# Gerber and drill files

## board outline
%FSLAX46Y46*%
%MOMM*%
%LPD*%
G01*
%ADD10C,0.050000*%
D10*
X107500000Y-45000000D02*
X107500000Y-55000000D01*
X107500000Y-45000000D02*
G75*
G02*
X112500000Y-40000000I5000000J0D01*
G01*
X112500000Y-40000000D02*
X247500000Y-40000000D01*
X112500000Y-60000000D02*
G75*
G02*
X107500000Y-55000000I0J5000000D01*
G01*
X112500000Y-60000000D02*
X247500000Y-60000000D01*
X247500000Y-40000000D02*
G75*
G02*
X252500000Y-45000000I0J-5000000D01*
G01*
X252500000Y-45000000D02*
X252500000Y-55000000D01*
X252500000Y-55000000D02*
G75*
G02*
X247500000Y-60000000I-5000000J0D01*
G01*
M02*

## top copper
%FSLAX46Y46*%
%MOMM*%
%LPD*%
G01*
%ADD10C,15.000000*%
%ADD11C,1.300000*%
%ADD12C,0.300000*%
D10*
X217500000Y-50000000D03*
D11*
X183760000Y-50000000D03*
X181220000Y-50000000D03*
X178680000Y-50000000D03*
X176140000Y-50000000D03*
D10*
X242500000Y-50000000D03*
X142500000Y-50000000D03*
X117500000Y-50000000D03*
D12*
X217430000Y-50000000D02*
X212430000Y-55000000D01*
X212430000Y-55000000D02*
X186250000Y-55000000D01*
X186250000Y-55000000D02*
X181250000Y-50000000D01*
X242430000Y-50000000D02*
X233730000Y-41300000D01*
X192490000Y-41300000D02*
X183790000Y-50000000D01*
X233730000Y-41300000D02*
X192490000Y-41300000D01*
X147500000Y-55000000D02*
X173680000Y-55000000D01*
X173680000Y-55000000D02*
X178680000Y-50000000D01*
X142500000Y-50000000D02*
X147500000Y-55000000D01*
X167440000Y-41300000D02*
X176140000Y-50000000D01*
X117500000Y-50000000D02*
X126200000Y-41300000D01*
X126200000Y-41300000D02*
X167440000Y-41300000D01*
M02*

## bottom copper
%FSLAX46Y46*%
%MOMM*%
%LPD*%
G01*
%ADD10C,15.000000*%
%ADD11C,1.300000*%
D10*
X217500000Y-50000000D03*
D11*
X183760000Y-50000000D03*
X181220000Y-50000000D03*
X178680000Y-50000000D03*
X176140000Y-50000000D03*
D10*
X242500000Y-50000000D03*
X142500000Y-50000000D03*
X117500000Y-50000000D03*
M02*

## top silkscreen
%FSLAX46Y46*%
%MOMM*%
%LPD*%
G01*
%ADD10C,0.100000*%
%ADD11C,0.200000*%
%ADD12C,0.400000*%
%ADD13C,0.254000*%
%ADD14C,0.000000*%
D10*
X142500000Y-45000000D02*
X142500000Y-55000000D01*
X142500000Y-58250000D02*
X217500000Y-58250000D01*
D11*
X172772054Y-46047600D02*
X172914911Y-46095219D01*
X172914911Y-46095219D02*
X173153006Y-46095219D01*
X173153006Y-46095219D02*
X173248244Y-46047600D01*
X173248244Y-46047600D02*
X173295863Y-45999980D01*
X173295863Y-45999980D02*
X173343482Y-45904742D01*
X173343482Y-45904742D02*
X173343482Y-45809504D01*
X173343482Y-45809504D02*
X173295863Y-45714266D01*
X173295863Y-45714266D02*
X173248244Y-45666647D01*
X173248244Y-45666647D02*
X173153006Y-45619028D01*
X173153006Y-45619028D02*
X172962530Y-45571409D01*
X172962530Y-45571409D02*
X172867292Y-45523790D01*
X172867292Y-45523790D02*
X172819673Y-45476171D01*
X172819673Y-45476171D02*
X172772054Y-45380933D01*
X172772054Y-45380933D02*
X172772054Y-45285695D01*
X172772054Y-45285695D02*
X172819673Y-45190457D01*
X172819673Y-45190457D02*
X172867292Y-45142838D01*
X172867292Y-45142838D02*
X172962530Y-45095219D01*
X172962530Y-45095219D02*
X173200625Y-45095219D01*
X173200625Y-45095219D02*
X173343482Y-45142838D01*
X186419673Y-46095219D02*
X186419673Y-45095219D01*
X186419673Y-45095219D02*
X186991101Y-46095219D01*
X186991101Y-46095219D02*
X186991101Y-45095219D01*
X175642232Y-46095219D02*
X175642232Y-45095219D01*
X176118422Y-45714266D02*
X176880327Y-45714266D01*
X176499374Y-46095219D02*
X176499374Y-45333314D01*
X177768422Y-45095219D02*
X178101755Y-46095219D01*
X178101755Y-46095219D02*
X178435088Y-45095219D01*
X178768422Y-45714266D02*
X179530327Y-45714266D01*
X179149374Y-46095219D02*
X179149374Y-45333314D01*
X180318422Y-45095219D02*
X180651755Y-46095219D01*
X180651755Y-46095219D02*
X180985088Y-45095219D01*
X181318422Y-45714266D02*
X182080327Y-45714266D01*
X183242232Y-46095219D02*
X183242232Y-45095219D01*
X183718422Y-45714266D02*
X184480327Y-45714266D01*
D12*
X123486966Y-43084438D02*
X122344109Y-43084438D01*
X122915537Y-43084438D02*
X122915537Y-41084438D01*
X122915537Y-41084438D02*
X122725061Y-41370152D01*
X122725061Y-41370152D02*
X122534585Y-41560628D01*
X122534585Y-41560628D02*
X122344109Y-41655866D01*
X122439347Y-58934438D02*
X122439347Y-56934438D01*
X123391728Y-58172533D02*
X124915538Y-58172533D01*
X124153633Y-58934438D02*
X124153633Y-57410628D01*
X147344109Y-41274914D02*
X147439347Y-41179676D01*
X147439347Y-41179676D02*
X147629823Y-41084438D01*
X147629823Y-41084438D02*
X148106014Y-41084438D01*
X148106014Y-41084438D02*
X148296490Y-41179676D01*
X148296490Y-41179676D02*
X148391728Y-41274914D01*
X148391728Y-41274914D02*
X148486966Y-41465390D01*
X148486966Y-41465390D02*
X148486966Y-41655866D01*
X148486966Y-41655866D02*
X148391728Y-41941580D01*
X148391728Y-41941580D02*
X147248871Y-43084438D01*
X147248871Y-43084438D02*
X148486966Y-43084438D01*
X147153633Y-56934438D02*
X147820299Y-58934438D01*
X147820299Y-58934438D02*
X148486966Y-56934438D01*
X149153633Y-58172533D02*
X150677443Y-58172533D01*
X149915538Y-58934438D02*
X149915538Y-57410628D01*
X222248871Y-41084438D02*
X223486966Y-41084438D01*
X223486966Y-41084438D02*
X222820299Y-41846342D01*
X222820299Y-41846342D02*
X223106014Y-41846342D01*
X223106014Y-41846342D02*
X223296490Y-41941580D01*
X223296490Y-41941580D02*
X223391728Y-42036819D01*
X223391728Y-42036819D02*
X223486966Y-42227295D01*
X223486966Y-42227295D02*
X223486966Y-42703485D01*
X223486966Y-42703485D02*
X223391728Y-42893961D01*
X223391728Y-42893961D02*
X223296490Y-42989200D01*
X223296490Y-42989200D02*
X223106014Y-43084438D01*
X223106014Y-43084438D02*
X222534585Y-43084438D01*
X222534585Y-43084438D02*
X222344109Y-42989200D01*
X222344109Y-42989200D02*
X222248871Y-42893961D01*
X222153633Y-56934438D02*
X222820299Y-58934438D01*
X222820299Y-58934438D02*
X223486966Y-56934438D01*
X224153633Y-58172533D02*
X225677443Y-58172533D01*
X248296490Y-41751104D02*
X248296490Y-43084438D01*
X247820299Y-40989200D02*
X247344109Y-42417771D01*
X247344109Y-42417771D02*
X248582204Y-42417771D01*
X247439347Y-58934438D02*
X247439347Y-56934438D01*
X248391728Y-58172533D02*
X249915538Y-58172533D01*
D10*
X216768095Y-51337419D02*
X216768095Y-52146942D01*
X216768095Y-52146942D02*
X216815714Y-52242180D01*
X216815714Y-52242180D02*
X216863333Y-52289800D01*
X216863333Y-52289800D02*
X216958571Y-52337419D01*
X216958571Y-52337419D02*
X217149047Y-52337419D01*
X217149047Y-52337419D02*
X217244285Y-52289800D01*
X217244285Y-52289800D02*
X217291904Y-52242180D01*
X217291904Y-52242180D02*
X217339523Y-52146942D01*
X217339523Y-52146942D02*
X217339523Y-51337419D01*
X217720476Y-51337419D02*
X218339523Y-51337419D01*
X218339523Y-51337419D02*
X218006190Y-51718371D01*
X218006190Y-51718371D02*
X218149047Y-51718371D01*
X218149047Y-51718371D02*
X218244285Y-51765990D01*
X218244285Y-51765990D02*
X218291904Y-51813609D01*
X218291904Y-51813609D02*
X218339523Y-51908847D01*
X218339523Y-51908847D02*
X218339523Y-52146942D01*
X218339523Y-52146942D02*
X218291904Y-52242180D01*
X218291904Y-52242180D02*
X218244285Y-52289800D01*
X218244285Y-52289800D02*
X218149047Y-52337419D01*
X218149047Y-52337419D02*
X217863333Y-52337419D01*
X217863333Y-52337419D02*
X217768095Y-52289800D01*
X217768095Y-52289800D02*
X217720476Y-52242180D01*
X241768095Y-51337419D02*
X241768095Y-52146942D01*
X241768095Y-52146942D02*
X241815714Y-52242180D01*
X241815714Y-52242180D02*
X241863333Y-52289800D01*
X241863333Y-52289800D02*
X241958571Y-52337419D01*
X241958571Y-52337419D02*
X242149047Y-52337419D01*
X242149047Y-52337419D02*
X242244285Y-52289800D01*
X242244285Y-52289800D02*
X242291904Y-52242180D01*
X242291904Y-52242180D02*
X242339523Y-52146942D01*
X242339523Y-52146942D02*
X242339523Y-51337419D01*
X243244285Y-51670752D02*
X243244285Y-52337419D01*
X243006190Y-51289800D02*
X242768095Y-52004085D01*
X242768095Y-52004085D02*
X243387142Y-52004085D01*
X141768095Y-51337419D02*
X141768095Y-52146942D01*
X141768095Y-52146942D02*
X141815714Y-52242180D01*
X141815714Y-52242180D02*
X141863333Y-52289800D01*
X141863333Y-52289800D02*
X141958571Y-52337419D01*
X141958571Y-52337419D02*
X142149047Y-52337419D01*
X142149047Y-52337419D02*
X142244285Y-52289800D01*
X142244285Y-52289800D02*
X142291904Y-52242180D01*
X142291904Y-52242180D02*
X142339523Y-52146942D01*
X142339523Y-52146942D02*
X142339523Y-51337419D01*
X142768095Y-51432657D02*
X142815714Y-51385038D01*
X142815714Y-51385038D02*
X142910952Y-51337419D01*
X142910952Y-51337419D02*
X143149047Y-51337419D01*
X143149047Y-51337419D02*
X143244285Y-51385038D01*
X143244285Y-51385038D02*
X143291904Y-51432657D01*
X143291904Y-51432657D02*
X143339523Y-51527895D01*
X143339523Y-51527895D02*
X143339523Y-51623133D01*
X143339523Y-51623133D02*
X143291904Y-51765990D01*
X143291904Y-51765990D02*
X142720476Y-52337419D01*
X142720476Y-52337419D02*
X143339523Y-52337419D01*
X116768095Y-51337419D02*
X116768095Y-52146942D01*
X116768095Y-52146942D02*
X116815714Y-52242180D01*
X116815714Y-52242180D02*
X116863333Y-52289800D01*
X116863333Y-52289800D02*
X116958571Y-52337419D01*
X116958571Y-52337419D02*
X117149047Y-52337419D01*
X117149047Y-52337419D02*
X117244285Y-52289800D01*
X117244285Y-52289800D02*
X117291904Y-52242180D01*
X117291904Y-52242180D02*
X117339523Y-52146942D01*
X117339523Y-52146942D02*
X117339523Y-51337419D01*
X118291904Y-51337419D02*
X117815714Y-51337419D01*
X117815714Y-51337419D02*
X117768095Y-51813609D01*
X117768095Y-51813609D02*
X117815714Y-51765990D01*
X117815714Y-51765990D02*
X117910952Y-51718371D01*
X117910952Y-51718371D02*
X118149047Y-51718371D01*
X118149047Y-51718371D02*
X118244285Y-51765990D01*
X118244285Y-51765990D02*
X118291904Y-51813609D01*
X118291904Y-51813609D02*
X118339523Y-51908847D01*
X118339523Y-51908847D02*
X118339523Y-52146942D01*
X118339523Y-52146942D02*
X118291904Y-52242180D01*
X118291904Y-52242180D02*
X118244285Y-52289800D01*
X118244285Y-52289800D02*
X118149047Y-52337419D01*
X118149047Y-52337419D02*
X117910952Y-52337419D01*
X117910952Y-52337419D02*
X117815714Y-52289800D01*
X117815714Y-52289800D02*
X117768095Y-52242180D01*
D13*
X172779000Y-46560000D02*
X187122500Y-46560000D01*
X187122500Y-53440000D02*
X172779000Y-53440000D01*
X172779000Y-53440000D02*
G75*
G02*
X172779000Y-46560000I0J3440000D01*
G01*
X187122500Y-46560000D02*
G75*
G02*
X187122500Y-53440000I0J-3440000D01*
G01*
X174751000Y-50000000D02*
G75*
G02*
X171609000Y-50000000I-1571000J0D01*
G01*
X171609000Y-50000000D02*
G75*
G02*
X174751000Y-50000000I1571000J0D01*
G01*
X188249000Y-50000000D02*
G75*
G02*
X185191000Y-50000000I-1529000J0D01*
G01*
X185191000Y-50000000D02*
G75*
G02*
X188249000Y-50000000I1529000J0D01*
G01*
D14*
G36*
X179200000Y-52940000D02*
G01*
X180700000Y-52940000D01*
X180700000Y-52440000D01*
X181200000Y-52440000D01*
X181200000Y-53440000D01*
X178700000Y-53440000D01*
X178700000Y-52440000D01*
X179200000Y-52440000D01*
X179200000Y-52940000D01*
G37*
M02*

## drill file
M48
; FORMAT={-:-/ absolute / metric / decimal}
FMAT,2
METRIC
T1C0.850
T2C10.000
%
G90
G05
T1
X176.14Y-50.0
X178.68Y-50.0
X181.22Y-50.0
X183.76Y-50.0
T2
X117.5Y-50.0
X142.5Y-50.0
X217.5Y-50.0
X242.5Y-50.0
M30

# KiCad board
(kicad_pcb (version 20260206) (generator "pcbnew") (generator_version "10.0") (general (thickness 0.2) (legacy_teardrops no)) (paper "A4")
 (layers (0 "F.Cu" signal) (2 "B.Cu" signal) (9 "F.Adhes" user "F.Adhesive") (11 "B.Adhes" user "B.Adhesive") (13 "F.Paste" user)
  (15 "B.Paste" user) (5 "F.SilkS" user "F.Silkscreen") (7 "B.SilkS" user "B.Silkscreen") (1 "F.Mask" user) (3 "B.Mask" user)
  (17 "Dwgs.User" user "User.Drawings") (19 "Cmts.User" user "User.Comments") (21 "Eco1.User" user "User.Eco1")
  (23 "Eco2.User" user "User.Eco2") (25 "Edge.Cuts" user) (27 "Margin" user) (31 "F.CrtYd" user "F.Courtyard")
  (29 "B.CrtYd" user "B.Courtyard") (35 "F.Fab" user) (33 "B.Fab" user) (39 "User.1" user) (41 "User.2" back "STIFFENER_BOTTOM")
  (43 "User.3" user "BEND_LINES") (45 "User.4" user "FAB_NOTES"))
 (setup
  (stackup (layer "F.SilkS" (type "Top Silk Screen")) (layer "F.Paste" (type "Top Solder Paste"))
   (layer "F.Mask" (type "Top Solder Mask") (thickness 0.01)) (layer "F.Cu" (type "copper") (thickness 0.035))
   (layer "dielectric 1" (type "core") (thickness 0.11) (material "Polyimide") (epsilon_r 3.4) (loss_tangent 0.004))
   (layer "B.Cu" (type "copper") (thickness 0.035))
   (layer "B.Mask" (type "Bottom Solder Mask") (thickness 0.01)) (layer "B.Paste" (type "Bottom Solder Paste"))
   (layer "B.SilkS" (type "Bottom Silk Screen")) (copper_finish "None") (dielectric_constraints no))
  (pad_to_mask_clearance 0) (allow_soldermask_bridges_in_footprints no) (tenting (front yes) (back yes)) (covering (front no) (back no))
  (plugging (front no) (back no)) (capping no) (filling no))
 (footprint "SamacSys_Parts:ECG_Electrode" (layer "F.Cu") (at 217.53 52.38)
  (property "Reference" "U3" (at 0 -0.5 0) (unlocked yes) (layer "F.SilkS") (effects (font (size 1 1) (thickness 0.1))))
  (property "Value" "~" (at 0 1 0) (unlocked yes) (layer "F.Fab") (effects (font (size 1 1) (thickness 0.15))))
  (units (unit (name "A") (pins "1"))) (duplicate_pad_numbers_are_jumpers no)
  (pad "1" thru_hole circle (at -0.03 -2.38) (size 15 15) (drill 10) (layers "*.Cu" "*.Mask") (remove_unused_layers no) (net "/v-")))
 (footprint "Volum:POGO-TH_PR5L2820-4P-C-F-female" (layer "F.Cu") (at 179.95 50 180)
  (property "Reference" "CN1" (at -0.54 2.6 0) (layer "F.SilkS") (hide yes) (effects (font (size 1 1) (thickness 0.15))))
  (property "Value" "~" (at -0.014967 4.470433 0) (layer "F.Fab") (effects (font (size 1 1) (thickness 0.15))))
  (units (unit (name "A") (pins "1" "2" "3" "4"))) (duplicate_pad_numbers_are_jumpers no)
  (fp_line (start 7.171 3.44) (end -7.1725 3.44) (stroke (width 0.254) (type default)) (layer "F.SilkS"))
  (fp_line (start -7.1725 -3.44) (end 7.171 -3.44) (stroke (width 0.254) (type default)) (layer "F.SilkS"))
  (fp_arc (start 7.171 -3.44) (mid 10.611 0) (end 7.171 3.44) (stroke (width 0.254) (type default)) (layer "F.SilkS"))
  (fp_arc (start -7.1725 3.44) (mid -10.6125 0) (end -7.1725 -3.44) (stroke (width 0.254) (type default)) (layer "F.SilkS"))
  (fp_circle (center 6.77 0) (end 8.341 0) (stroke (width 0.254) (type default)) (fill no) (layer "F.SilkS"))
  (fp_circle (center -6.77 0) (end -5.241 0) (stroke (width 0.254) (type default)) (fill no) (layer "F.SilkS"))
  (fp_poly
   (pts (xy 1.25 -2.44) (xy 1.25 -3.44) (xy -1.25 -3.44) (xy -1.25 -2.44) (xy -0.75 -2.44) (xy -0.75 -2.94) (xy 0.75 -2.94) (xy 0.75 -2.44))
   (stroke (width 0) (type default)) (fill yes) (layer "F.SilkS"))
  (pad "1" thru_hole circle (at -3.81 0 180) (size 1.3 1.3) (drill 0.85) (layers "*.Cu" "*.Mask") (remove_unused_layers no) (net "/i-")
   (thermal_bridge_angle 90))
  (pad "2" thru_hole circle (at -1.27 0 180) (size 1.3 1.3) (drill 0.85) (layers "*.Cu" "*.Mask") (remove_unused_layers no) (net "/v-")
   (thermal_bridge_angle 90))
  (pad "3" thru_hole circle (at 1.27 0 180) (size 1.3 1.3) (drill 0.85) (layers "*.Cu" "*.Mask") (remove_unused_layers no) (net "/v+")
   (thermal_bridge_angle 90))
  (pad "4" thru_hole circle (at 3.81 0 180) (size 1.3 1.3) (drill 0.85) (layers "*.Cu" "*.Mask") (remove_unused_layers no) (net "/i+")
   (thermal_bridge_angle 90)))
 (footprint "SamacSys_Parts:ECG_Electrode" (layer "F.Cu") (at 242.53 52.38)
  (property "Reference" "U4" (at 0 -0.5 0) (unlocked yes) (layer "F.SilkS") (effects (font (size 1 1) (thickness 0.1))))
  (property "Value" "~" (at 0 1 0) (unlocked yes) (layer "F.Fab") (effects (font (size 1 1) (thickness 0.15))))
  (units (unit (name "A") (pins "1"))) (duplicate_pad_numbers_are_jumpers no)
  (pad "1" thru_hole circle (at -0.03 -2.38) (size 15 15) (drill 10) (layers "*.Cu" "*.Mask") (remove_unused_layers no) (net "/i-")))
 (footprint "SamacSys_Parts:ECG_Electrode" (layer "F.Cu") (at 142.53 52.38)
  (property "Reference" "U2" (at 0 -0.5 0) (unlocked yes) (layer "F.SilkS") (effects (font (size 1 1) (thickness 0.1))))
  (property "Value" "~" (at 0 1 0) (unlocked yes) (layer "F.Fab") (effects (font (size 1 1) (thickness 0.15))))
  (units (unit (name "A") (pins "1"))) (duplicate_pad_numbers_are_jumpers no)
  (pad "1" thru_hole circle (at -0.03 -2.38) (size 15 15) (drill 10) (layers "*.Cu" "*.Mask") (remove_unused_layers no) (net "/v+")))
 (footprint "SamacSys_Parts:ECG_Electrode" (layer "F.Cu") (at 117.53 52.38)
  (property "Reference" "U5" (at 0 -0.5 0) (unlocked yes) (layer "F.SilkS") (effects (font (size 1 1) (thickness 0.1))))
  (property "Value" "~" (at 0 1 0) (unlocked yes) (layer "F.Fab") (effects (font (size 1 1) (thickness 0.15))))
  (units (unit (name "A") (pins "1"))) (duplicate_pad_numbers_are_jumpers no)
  (pad "1" thru_hole circle (at -0.03 -2.38) (size 15 15) (drill 10) (layers "*.Cu" "*.Mask") (remove_unused_layers no) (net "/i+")))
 (gr_line (start 142.5 45) (end 142.5 55) (stroke (width 0.1) (type default)) (layer "F.SilkS"))
 (gr_line (start 142.5 58.25) (end 217.5 58.25) (stroke (width 0.1) (type default)) (layer "F.SilkS"))
 (gr_line (start 107.5 45) (end 107.5 55) (stroke (width 0.05) (type default)) (layer "Edge.Cuts"))
 (gr_arc (start 107.5 45) (mid 108.964466 41.464466) (end 112.5 40) (stroke (width 0.05) (type default)) (layer "Edge.Cuts"))
 (gr_line (start 112.5 40) (end 247.5 40) (stroke (width 0.05) (type default)) (layer "Edge.Cuts"))
 (gr_arc (start 112.5 60) (mid 108.964466 58.535534) (end 107.5 55) (stroke (width 0.05) (type default)) (layer "Edge.Cuts"))
 (gr_line (start 112.5 60) (end 247.5 60) (stroke (width 0.05) (type default)) (layer "Edge.Cuts"))
 (gr_arc (start 247.5 40) (mid 251.035534 41.464466) (end 252.5 45) (stroke (width 0.05) (type default)) (layer "Edge.Cuts"))
 (gr_line (start 252.5 45) (end 252.5 55) (stroke (width 0.05) (type default)) (layer "Edge.Cuts"))
 (gr_arc (start 252.5 55) (mid 251.035534 58.535534) (end 247.5 60) (stroke (width 0.05) (type default)) (layer "Edge.Cuts"))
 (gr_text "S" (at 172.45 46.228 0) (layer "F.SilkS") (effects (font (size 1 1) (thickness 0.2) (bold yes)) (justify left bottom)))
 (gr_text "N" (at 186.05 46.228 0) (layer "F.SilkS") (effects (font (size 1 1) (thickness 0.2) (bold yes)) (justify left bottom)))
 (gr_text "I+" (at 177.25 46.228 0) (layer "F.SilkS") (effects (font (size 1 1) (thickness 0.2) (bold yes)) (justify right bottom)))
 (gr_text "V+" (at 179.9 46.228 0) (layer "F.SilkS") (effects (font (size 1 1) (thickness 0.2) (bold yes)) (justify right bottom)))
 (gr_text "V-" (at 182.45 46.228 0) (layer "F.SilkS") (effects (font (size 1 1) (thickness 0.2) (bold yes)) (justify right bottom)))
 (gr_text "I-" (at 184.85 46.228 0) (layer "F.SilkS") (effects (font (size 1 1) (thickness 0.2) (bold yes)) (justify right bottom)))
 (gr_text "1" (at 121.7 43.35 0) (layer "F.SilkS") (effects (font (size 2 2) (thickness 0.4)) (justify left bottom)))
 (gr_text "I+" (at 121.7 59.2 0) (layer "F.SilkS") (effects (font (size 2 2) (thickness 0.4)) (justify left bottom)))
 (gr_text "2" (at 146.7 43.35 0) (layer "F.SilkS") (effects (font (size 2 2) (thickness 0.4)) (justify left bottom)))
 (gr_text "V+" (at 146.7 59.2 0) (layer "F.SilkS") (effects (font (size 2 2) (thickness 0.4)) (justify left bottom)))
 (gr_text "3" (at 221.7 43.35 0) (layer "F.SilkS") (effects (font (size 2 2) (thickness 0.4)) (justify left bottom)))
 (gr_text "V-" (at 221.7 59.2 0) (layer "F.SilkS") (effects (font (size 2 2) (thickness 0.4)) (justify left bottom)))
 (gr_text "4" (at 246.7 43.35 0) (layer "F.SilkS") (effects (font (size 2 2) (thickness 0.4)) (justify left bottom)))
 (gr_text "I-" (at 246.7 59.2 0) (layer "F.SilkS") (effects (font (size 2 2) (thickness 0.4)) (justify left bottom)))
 (segment (start 217.43 50) (end 212.43 55) (width 0.3) (layer "F.Cu") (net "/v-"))
 (segment (start 212.43 55) (end 186.25 55) (width 0.3) (layer "F.Cu") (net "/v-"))
 (segment (start 186.25 55) (end 181.25 50) (width 0.3) (layer "F.Cu") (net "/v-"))
 (segment (start 242.43 50) (end 233.73 41.3) (width 0.3) (layer "F.Cu") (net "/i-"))
 (segment (start 192.49 41.3) (end 183.79 50) (width 0.3) (layer "F.Cu") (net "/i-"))
 (segment (start 233.73 41.3) (end 192.49 41.3) (width 0.3) (layer "F.Cu") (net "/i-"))
 (segment (start 147.5 55) (end 173.68 55) (width 0.3) (layer "F.Cu") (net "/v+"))
 (segment (start 173.68 55) (end 178.68 50) (width 0.3) (layer "F.Cu") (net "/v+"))
 (segment (start 142.5 50) (end 147.5 55) (width 0.3) (layer "F.Cu") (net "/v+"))
 (segment (start 167.44 41.3) (end 176.14 50) (width 0.3) (layer "F.Cu") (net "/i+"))
 (segment (start 117.5 50) (end 126.2 41.3) (width 0.3) (layer "F.Cu") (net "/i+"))
 (segment (start 126.2 41.3) (end 167.44 41.3) (width 0.3) (layer "F.Cu") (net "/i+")))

